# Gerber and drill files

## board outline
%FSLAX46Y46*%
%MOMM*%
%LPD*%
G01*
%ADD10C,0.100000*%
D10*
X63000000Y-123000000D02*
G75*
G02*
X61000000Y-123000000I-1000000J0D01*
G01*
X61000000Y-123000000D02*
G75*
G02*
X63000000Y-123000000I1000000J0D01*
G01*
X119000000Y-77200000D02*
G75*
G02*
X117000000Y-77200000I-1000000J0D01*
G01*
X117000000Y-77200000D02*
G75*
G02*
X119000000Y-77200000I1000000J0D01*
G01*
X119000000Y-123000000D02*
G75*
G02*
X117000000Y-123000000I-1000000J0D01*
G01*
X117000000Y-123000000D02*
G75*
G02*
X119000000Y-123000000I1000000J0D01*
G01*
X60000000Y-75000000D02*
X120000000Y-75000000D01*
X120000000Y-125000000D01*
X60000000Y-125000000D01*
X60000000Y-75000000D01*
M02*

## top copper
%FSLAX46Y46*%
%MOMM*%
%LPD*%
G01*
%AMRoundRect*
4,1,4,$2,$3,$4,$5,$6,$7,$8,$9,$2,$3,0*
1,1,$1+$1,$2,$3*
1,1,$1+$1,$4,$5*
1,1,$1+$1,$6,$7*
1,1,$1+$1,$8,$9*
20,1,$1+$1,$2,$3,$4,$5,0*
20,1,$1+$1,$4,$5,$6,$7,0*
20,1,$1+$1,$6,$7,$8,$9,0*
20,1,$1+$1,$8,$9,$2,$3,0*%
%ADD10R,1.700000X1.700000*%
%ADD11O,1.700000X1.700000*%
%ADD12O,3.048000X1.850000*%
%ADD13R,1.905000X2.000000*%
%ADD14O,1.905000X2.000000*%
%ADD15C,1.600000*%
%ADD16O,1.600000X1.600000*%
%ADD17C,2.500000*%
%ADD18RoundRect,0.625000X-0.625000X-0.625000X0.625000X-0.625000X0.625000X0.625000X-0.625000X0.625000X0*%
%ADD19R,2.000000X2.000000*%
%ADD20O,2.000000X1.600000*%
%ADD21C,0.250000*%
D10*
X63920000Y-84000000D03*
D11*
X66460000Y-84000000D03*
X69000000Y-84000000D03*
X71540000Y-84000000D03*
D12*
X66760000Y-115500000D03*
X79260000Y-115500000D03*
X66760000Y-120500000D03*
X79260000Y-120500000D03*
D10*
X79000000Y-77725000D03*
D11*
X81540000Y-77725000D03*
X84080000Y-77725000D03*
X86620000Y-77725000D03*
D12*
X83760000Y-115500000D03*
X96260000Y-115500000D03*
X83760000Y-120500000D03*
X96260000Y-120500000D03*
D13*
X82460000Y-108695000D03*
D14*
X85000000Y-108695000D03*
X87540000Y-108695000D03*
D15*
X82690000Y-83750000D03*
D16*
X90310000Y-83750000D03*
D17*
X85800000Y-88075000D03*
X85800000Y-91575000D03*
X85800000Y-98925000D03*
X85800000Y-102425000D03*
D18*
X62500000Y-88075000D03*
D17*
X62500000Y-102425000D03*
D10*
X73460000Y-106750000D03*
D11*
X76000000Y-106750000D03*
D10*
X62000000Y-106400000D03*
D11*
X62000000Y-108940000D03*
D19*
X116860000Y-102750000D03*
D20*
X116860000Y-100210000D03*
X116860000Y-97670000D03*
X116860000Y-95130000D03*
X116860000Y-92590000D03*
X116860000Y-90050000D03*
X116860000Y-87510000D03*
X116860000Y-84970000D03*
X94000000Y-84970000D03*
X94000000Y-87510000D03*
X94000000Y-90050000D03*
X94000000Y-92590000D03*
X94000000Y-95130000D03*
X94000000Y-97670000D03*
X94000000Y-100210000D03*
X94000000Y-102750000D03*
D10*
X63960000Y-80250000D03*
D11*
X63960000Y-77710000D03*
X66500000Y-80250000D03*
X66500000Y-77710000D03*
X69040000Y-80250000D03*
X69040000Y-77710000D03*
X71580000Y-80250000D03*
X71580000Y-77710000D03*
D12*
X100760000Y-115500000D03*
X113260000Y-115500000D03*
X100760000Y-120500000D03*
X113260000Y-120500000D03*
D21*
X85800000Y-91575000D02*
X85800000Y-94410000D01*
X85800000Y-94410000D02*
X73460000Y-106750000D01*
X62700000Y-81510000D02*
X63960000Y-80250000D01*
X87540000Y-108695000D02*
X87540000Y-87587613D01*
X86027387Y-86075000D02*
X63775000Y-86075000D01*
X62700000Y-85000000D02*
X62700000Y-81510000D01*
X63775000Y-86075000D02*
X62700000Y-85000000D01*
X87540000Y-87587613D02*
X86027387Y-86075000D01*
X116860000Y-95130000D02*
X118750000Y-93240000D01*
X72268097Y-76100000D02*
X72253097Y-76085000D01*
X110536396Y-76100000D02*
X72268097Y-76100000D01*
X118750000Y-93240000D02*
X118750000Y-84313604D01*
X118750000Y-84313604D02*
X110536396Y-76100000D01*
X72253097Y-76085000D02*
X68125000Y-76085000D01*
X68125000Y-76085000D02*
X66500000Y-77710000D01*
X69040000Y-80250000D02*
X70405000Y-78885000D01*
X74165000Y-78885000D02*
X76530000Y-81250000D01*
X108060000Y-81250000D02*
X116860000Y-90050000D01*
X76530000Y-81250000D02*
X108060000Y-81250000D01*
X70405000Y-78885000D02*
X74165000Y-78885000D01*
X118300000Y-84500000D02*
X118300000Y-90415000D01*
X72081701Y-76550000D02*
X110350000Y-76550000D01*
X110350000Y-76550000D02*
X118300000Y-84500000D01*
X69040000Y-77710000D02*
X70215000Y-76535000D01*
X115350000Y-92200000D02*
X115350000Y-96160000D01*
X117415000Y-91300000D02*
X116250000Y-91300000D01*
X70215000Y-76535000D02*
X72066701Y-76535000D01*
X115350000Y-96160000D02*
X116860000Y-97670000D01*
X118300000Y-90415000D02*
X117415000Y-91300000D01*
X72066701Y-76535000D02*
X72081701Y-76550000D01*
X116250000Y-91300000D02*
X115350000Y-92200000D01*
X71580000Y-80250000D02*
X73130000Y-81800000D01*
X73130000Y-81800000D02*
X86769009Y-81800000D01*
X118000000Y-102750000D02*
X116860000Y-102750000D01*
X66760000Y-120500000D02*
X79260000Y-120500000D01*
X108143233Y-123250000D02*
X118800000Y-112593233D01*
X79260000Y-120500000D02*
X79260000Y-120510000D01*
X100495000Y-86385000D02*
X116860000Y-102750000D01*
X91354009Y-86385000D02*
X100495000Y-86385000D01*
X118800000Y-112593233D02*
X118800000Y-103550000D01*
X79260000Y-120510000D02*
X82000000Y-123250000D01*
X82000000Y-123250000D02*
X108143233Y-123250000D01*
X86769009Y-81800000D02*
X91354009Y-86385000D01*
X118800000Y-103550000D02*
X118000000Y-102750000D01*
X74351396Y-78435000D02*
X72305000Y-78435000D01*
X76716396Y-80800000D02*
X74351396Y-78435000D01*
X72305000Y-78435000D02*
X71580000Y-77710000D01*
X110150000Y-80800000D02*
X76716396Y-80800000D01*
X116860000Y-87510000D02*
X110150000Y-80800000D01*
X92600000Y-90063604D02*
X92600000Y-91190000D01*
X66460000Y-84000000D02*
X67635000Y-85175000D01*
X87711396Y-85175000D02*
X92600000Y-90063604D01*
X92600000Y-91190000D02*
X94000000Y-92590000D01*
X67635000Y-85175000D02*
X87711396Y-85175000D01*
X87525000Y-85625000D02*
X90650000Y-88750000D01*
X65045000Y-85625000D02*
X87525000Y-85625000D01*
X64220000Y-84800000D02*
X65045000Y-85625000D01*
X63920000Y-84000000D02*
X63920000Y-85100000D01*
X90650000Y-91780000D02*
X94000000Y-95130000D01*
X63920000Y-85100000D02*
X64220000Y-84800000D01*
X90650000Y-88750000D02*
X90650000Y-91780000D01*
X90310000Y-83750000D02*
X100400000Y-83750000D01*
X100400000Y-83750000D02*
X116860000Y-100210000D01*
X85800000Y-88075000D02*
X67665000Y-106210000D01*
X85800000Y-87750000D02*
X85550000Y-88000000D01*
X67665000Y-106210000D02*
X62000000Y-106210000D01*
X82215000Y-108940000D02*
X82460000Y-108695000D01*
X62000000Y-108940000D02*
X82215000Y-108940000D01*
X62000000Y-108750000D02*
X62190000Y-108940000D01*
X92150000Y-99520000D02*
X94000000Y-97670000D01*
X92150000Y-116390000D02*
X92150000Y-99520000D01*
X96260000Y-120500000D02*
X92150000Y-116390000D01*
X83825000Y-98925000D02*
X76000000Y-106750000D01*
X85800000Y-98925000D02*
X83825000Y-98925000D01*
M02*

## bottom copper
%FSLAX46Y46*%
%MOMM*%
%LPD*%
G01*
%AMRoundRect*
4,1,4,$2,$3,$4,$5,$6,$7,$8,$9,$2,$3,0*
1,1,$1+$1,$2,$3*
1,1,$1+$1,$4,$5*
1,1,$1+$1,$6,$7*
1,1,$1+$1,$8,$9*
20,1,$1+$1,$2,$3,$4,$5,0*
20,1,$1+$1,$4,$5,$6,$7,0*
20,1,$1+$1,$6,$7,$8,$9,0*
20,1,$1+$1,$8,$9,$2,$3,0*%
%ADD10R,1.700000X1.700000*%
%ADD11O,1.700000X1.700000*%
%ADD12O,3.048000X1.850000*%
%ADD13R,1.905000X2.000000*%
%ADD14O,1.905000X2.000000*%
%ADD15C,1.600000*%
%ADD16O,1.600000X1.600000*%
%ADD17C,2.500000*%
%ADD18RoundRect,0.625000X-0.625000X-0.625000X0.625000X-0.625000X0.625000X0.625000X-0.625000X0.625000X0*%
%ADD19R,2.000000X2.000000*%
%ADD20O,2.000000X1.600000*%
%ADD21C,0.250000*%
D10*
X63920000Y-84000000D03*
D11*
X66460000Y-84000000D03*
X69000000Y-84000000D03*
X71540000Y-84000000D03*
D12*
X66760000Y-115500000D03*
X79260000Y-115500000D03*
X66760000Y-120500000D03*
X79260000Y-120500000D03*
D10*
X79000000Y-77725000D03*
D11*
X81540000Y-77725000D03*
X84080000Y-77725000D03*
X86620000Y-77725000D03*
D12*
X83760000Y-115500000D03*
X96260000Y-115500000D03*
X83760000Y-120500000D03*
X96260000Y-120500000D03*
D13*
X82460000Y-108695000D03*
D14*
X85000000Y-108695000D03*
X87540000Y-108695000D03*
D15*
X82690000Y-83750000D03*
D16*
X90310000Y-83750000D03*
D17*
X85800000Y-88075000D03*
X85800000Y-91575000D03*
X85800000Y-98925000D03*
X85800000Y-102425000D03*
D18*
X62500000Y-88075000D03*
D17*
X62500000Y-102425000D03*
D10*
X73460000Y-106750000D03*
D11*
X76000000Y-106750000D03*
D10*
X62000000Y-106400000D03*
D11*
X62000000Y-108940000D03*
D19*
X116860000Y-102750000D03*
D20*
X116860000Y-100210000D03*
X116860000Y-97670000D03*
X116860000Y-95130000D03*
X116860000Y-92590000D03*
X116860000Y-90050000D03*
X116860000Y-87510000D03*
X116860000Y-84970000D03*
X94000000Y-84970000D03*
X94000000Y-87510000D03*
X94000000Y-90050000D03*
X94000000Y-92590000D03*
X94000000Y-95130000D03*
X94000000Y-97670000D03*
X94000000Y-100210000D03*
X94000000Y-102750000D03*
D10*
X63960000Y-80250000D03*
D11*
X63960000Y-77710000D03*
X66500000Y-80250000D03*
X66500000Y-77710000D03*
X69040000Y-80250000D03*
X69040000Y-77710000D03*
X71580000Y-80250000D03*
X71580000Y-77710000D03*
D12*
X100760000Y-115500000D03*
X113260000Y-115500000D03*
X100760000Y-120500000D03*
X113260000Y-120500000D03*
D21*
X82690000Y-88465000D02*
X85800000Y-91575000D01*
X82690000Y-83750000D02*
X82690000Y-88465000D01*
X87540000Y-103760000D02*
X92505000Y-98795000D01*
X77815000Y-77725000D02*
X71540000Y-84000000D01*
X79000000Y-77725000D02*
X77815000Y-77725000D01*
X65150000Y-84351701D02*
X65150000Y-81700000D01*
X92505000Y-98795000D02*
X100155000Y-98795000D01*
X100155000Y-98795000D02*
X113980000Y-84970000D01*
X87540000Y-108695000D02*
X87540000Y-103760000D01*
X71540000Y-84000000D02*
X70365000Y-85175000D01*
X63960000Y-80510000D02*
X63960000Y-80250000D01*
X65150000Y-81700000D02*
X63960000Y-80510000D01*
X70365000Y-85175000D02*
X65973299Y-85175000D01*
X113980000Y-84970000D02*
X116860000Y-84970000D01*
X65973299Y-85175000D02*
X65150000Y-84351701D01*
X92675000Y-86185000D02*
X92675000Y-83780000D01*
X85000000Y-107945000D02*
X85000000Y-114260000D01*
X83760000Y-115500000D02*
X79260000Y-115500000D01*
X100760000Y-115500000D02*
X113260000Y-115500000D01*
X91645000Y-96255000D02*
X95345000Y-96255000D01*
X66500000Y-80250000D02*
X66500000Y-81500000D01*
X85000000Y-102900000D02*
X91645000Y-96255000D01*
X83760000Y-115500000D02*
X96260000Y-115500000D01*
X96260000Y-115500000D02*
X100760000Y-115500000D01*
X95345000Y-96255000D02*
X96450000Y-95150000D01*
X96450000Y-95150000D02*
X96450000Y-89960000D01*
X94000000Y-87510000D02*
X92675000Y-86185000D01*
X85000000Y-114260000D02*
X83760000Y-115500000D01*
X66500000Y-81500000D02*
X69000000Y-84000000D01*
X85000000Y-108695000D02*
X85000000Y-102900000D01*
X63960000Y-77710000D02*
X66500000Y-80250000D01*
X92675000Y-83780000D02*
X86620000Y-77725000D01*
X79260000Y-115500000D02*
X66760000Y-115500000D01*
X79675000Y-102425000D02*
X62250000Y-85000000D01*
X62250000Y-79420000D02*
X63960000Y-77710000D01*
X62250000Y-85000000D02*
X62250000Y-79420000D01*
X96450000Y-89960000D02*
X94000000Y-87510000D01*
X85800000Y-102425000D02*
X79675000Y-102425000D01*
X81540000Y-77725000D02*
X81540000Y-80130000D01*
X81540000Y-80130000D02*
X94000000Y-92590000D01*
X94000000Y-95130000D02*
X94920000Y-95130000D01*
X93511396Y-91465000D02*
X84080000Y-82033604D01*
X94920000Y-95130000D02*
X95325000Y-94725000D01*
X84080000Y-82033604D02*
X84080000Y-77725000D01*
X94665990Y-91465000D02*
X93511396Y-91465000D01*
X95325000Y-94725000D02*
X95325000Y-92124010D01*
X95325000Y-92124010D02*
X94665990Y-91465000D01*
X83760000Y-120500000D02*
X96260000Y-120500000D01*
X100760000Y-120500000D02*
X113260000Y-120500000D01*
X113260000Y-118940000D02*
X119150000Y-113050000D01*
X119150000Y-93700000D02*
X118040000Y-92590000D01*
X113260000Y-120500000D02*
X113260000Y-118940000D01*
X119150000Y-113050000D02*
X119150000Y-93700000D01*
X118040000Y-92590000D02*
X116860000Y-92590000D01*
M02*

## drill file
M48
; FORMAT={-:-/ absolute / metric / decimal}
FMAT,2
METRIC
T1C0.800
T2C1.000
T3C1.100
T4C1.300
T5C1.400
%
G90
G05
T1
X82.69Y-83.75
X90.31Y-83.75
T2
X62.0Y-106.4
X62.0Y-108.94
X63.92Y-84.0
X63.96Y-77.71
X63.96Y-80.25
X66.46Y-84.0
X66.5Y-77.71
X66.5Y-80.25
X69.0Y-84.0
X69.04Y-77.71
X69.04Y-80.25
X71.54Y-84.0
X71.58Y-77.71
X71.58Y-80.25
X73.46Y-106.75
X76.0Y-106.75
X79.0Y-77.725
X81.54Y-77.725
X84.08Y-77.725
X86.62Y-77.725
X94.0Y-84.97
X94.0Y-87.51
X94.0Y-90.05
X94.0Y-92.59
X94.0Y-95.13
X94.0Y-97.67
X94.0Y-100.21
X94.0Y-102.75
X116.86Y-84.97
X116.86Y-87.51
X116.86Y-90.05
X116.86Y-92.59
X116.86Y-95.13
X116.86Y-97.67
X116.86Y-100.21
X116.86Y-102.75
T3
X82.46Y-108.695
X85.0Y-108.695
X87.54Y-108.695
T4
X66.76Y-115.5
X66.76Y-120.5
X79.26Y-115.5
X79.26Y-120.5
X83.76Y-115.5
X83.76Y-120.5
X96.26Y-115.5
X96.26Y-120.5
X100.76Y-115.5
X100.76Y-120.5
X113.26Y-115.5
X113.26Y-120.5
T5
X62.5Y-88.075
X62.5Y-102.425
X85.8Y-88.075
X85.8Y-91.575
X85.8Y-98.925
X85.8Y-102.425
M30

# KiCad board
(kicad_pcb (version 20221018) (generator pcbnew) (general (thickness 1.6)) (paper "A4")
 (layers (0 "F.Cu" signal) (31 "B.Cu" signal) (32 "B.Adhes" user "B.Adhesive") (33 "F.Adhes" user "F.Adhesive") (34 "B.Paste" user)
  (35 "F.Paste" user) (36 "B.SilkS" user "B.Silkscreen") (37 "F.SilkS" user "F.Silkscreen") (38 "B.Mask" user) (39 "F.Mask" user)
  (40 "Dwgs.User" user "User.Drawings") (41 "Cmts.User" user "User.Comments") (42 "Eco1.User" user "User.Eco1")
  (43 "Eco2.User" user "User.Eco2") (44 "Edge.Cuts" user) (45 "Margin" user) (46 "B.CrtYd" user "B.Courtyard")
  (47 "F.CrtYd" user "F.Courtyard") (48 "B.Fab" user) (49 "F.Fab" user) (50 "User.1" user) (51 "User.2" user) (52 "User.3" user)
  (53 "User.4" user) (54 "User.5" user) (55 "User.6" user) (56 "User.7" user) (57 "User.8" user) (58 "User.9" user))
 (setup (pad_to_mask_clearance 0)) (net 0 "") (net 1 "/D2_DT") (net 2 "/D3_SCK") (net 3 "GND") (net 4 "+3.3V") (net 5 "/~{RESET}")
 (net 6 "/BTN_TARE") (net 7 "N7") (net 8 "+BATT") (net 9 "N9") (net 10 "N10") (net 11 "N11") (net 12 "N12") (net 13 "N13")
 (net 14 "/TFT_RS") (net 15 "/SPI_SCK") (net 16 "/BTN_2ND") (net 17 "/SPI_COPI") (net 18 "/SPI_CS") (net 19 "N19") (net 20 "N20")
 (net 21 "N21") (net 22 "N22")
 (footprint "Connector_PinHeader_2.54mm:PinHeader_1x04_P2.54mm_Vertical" (layer "F.Cu") (at 63.92 84 90)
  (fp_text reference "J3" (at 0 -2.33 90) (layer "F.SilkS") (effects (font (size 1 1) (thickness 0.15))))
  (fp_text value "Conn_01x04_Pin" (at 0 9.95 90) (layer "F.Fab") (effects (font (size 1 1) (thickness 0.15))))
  (pad "1" thru_hole rect (at 0 0 90) (size 1.7 1.7) (drill 1) (layers "*.Cu" "*.Mask") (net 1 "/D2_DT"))
  (pad "2" thru_hole oval (at 0 2.54 90) (size 1.7 1.7) (drill 1) (layers "*.Cu" "*.Mask") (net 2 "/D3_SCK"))
  (pad "3" thru_hole oval (at 0 5.08 90) (size 1.7 1.7) (drill 1) (layers "*.Cu" "*.Mask") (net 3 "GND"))
  (pad "4" thru_hole oval (at 0 7.62 90) (size 1.7 1.7) (drill 1) (layers "*.Cu" "*.Mask") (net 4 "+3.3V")))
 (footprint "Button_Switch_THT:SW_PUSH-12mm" (layer "F.Cu") (at 66.76 115.5)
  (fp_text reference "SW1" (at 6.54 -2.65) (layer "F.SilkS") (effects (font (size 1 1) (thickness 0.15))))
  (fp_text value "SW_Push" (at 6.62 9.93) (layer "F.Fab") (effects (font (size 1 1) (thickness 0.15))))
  (pad "1" thru_hole oval (at 0 0) (size 3.048 1.85) (drill 1.3) (layers "*.Cu" "*.Mask") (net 3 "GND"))
  (pad "1" thru_hole oval (at 12.5 0) (size 3.048 1.85) (drill 1.3) (layers "*.Cu" "*.Mask") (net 3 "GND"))
  (pad "2" thru_hole oval (at 0 5) (size 3.048 1.85) (drill 1.3) (layers "*.Cu" "*.Mask") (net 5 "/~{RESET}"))
  (pad "2" thru_hole oval (at 12.5 5) (size 3.048 1.85) (drill 1.3) (layers "*.Cu" "*.Mask") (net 5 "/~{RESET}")))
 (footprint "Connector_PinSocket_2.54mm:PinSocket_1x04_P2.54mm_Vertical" (layer "F.Cu") (at 79 77.725 90)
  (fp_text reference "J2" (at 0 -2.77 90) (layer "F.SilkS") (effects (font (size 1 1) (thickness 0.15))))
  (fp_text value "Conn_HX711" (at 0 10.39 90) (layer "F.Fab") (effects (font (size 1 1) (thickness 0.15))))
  (pad "1" thru_hole rect (at 0 0 90) (size 1.7 1.7) (drill 1) (layers "*.Cu" "*.Mask") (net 4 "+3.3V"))
  (pad "2" thru_hole oval (at 0 2.54 90) (size 1.7 1.7) (drill 1) (layers "*.Cu" "*.Mask") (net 2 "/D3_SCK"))
  (pad "3" thru_hole oval (at 0 5.08 90) (size 1.7 1.7) (drill 1) (layers "*.Cu" "*.Mask") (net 1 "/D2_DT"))
  (pad "4" thru_hole oval (at 0 7.62 90) (size 1.7 1.7) (drill 1) (layers "*.Cu" "*.Mask") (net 3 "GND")))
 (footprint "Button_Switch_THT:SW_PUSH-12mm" (layer "F.Cu") (at 83.76 115.5)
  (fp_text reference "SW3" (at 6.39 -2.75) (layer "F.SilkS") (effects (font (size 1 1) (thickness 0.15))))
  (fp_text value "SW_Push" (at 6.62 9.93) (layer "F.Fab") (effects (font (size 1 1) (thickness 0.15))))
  (pad "1" thru_hole oval (at 0 0) (size 3.048 1.85) (drill 1.3) (layers "*.Cu" "*.Mask") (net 3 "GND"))
  (pad "1" thru_hole oval (at 12.5 0) (size 3.048 1.85) (drill 1.3) (layers "*.Cu" "*.Mask") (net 3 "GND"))
  (pad "2" thru_hole oval (at 0 5) (size 3.048 1.85) (drill 1.3) (layers "*.Cu" "*.Mask") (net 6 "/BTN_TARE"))
  (pad "2" thru_hole oval (at 12.5 5) (size 3.048 1.85) (drill 1.3) (layers "*.Cu" "*.Mask") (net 6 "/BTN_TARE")))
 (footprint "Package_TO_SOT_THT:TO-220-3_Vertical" (layer "F.Cu") (at 82.46 108.695)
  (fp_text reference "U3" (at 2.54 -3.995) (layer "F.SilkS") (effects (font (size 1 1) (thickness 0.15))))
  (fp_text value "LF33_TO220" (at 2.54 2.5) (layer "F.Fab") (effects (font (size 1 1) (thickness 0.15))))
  (pad "1" thru_hole rect (at 0 0) (size 1.905 2) (drill 1.1) (layers "*.Cu" "*.Mask") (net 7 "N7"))
  (pad "2" thru_hole oval (at 2.54 0) (size 1.905 2) (drill 1.1) (layers "*.Cu" "*.Mask") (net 3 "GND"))
  (pad "3" thru_hole oval (at 5.08 0) (size 1.905 2) (drill 1.1) (layers "*.Cu" "*.Mask") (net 4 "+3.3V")))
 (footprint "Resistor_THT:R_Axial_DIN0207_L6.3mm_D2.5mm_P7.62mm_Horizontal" (layer "F.Cu") (at 82.69 83.75)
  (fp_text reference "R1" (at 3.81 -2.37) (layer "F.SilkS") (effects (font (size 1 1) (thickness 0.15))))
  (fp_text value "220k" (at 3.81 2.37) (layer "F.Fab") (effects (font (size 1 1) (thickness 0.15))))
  (pad "1" thru_hole circle (at 0 0) (size 1.6 1.6) (drill 0.8) (layers "*.Cu" "*.Mask") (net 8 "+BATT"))
  (pad "2" thru_hole oval (at 7.62 0) (size 1.6 1.6) (drill 0.8) (layers "*.Cu" "*.Mask") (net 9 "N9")))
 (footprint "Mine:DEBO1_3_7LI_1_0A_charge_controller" (layer "F.Cu") (at 60.8 93.575)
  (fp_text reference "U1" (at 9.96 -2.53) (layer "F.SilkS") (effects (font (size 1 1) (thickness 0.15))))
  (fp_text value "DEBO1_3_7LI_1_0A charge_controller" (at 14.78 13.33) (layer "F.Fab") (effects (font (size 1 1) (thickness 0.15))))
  (pad "1" thru_hole circle (at 25 -5.5) (size 2.5 2.5) (drill 1.4) (layers "*.Cu" "*.Mask") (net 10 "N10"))
  (pad "2" thru_hole circle (at 25 -2) (size 2.5 2.5) (drill 1.4) (layers "*.Cu" "*.Mask") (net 8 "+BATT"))
  (pad "3" thru_hole circle (at 25 5.35) (size 2.5 2.5) (drill 1.4) (layers "*.Cu" "*.Mask") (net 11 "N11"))
  (pad "4" thru_hole circle (at 25 8.85) (size 2.5 2.5) (drill 1.4) (layers "*.Cu" "*.Mask") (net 3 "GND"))
  (pad "5" thru_hole roundrect (at 1.7 -5.5) (size 2.5 2.5) (drill 1.4) (layers "*.Cu" "*.Mask") (roundrect_rratio 0.25) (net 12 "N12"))
  (pad "6" thru_hole circle (at 1.7 8.85) (size 2.5 2.5) (drill 1.4) (layers "*.Cu" "*.Mask") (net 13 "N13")))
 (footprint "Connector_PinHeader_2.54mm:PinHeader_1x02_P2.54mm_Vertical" (layer "F.Cu") (at 73.46 106.75 90)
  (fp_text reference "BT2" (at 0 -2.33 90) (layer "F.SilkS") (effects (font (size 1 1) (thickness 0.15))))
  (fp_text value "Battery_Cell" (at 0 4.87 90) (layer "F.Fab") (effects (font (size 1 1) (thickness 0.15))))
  (pad "1" thru_hole rect (at 0 0 90) (size 1.7 1.7) (drill 1) (layers "*.Cu" "*.Mask") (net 8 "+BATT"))
  (pad "2" thru_hole oval (at 0 2.54 90) (size 1.7 1.7) (drill 1) (layers "*.Cu" "*.Mask") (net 11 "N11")))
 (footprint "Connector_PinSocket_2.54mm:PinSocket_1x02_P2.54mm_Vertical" (layer "F.Cu") (at 62 106.4)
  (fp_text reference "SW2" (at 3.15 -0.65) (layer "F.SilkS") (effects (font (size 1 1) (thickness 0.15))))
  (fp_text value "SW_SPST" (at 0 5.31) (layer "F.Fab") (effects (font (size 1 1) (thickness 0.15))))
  (pad "1" thru_hole rect (at 0 0) (size 1.7 1.7) (drill 1) (layers "*.Cu" "*.Mask") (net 10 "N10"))
  (pad "2" thru_hole oval (at 0 2.54) (size 1.7 1.7) (drill 1) (layers "*.Cu" "*.Mask") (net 7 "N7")))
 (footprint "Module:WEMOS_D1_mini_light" (layer "F.Cu") (at 116.86 102.75 180)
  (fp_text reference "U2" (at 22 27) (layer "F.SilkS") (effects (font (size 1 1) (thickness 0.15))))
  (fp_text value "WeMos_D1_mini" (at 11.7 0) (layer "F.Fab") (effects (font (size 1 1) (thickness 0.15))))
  (pad "1" thru_hole rect (at 0 0 180) (size 2 2) (drill 1) (layers "*.Cu" "*.Mask") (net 5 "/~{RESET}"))
  (pad "2" thru_hole oval (at 0 2.54 180) (size 2 1.6) (drill 1) (layers "*.Cu" "*.Mask") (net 9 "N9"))
  (pad "3" thru_hole oval (at 0 5.08 180) (size 2 1.6) (drill 1) (layers "*.Cu" "*.Mask") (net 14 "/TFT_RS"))
  (pad "4" thru_hole oval (at 0 7.62 180) (size 2 1.6) (drill 1) (layers "*.Cu" "*.Mask") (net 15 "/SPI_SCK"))
  (pad "5" thru_hole oval (at 0 10.16 180) (size 2 1.6) (drill 1) (layers "*.Cu" "*.Mask") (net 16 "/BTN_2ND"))
  (pad "6" thru_hole oval (at 0 12.7 180) (size 2 1.6) (drill 1) (layers "*.Cu" "*.Mask") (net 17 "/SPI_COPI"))
  (pad "7" thru_hole oval (at 0 15.24 180) (size 2 1.6) (drill 1) (layers "*.Cu" "*.Mask") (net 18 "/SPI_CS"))
  (pad "8" thru_hole oval (at 0 17.78 180) (size 2 1.6) (drill 1) (layers "*.Cu" "*.Mask") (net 4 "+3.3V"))
  (pad "9" thru_hole oval (at 22.86 17.78 180) (size 2 1.6) (drill 1) (layers "*.Cu" "*.Mask") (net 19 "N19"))
  (pad "10" thru_hole oval (at 22.86 15.24 180) (size 2 1.6) (drill 1) (layers "*.Cu" "*.Mask") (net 3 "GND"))
  (pad "11" thru_hole oval (at 22.86 12.7 180) (size 2 1.6) (drill 1) (layers "*.Cu" "*.Mask") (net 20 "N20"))
  (pad "12" thru_hole oval (at 22.86 10.16 180) (size 2 1.6) (drill 1) (layers "*.Cu" "*.Mask") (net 2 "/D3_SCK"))
  (pad "13" thru_hole oval (at 22.86 7.62 180) (size 2 1.6) (drill 1) (layers "*.Cu" "*.Mask") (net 1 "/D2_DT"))
  (pad "14" thru_hole oval (at 22.86 5.08 180) (size 2 1.6) (drill 1) (layers "*.Cu" "*.Mask") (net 6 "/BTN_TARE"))
  (pad "15" thru_hole oval (at 22.86 2.54 180) (size 2 1.6) (drill 1) (layers "*.Cu" "*.Mask") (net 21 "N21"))
  (pad "16" thru_hole oval (at 22.86 0 180) (size 2 1.6) (drill 1) (layers "*.Cu" "*.Mask") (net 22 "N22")))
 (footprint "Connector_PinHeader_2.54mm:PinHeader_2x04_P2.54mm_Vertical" (layer "F.Cu") (at 63.96 80.25 90)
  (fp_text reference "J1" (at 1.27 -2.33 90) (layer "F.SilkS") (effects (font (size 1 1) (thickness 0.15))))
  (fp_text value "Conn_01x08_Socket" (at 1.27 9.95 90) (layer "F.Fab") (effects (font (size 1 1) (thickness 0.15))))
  (pad "1" thru_hole rect (at 0 0 90) (size 1.7 1.7) (drill 1) (layers "*.Cu" "*.Mask") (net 4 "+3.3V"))
  (pad "2" thru_hole oval (at 2.54 0 90) (size 1.7 1.7) (drill 1) (layers "*.Cu" "*.Mask") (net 3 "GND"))
  (pad "3" thru_hole oval (at 0 2.54 90) (size 1.7 1.7) (drill 1) (layers "*.Cu" "*.Mask") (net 3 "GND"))
  (pad "4" thru_hole oval (at 2.54 2.54 90) (size 1.7 1.7) (drill 1) (layers "*.Cu" "*.Mask") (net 15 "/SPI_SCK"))
  (pad "5" thru_hole oval (at 0 5.08 90) (size 1.7 1.7) (drill 1) (layers "*.Cu" "*.Mask") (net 17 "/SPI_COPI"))
  (pad "6" thru_hole oval (at 2.54 5.08 90) (size 1.7 1.7) (drill 1) (layers "*.Cu" "*.Mask") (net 14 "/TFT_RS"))
  (pad "7" thru_hole oval (at 0 7.62 90) (size 1.7 1.7) (drill 1) (layers "*.Cu" "*.Mask") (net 5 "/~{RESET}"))
  (pad "8" thru_hole oval (at 2.54 7.62 90) (size 1.7 1.7) (drill 1) (layers "*.Cu" "*.Mask") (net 18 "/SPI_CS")))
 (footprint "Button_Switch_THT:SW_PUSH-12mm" (layer "F.Cu") (at 100.76 115.5)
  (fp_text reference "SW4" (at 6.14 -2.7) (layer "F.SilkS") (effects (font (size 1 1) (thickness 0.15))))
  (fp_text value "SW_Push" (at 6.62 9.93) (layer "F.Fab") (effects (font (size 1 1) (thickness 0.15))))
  (pad "1" thru_hole oval (at 0 0) (size 3.048 1.85) (drill 1.3) (layers "*.Cu" "*.Mask") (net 3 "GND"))
  (pad "1" thru_hole oval (at 12.5 0) (size 3.048 1.85) (drill 1.3) (layers "*.Cu" "*.Mask") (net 3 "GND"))
  (pad "2" thru_hole oval (at 0 5) (size 3.048 1.85) (drill 1.3) (layers "*.Cu" "*.Mask") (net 16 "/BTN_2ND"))
  (pad "2" thru_hole oval (at 12.5 5) (size 3.048 1.85) (drill 1.3) (layers "*.Cu" "*.Mask") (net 16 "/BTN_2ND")))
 (gr_circle (center 62 123) (end 62.8 123.6) (stroke (width 0.1) (type default)) (fill none) (layer "Edge.Cuts"))
 (gr_circle (center 118 77.2) (end 118.8 77.8) (stroke (width 0.1) (type default)) (fill none) (layer "Edge.Cuts"))
 (gr_circle (center 118 123) (end 118.8 123.6) (stroke (width 0.1) (type default)) (fill none) (layer "Edge.Cuts"))
 (gr_rect (start 60 75) (end 120 125) (stroke (width 0.1) (type default)) (fill none) (layer "Edge.Cuts"))
 (segment (start 85.8 91.575) (end 85.8 94.41) (width 0.25) (layer "F.Cu") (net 8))
 (segment (start 85.8 94.41) (end 73.46 106.75) (width 0.25) (layer "F.Cu") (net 8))
 (segment (start 82.69 88.465) (end 85.8 91.575) (width 0.25) (layer "B.Cu") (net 8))
 (segment (start 82.69 83.75) (end 82.69 88.465) (width 0.25) (layer "B.Cu") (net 8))
 (segment (start 62.7 81.51) (end 63.96 80.25) (width 0.25) (layer "F.Cu") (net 4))
 (segment (start 87.54 108.695) (end 87.54 87.587613) (width 0.25) (layer "F.Cu") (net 4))
 (segment (start 86.027387 86.075) (end 63.775 86.075) (width 0.25) (layer "F.Cu") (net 4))
 (segment (start 62.7 85) (end 62.7 81.51) (width 0.25) (layer "F.Cu") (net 4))
 (segment (start 63.775 86.075) (end 62.7 85) (width 0.25) (layer "F.Cu") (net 4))
 (segment (start 87.54 87.587613) (end 86.027387 86.075) (width 0.25) (layer "F.Cu") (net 4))
 (segment (start 87.54 103.76) (end 92.505 98.795) (width 0.25) (layer "B.Cu") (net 4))
 (segment (start 77.815 77.725) (end 71.54 84) (width 0.25) (layer "B.Cu") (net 4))
 (segment (start 79 77.725) (end 77.815 77.725) (width 0.25) (layer "B.Cu") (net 4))
 (segment (start 65.15 84.351701) (end 65.15 81.7) (width 0.25) (layer "B.Cu") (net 4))
 (segment (start 92.505 98.795) (end 100.155 98.795) (width 0.25) (layer "B.Cu") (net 4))
 (segment (start 100.155 98.795) (end 113.98 84.97) (width 0.25) (layer "B.Cu") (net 4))
 (segment (start 87.54 108.695) (end 87.54 103.76) (width 0.25) (layer "B.Cu") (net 4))
 (segment (start 71.54 84) (end 70.365 85.175) (width 0.25) (layer "B.Cu") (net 4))
 (segment (start 63.96 80.51) (end 63.96 80.25) (width 0.25) (layer "B.Cu") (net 4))
 (segment (start 65.15 81.7) (end 63.96 80.51) (width 0.25) (layer "B.Cu") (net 4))
 (segment (start 70.365 85.175) (end 65.973299 85.175) (width 0.25) (layer "B.Cu") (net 4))
 (segment (start 113.98 84.97) (end 116.86 84.97) (width 0.25) (layer "B.Cu") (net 4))
 (segment (start 65.973299 85.175) (end 65.15 84.351701) (width 0.25) (layer "B.Cu") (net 4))
 (segment (start 92.675 86.185) (end 92.675 83.78) (width 0.25) (layer "B.Cu") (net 3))
 (segment (start 85 107.945) (end 85 114.26) (width 0.25) (layer "B.Cu") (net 3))
 (segment (start 83.76 115.5) (end 79.26 115.5) (width 0.25) (layer "B.Cu") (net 3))
 (segment (start 100.76 115.5) (end 113.26 115.5) (width 0.25) (layer "B.Cu") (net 3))
 (segment (start 91.645 96.255) (end 95.345 96.255) (width 0.25) (layer "B.Cu") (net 3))
 (segment (start 66.5 80.25) (end 66.5 81.5) (width 0.25) (layer "B.Cu") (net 3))
 (segment (start 85 102.9) (end 91.645 96.255) (width 0.25) (layer "B.Cu") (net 3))
 (segment (start 83.76 115.5) (end 96.26 115.5) (width 0.25) (layer "B.Cu") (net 3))
 (segment (start 96.26 115.5) (end 100.76 115.5) (width 0.25) (layer "B.Cu") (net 3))
 (segment (start 95.345 96.255) (end 96.45 95.15) (width 0.25) (layer "B.Cu") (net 3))
 (segment (start 96.45 95.15) (end 96.45 89.96) (width 0.25) (layer "B.Cu") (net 3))
 (segment (start 94 87.51) (end 92.675 86.185) (width 0.25) (layer "B.Cu") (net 3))
 (segment (start 85 114.26) (end 83.76 115.5) (width 0.25) (layer "B.Cu") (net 3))
 (segment (start 66.5 81.5) (end 69 84) (width 0.25) (layer "B.Cu") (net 3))
 (segment (start 85 108.695) (end 85 102.9) (width 0.25) (layer "B.Cu") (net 3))
 (segment (start 63.96 77.71) (end 66.5 80.25) (width 0.25) (layer "B.Cu") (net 3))
 (segment (start 92.675 83.78) (end 86.62 77.725) (width 0.25) (layer "B.Cu") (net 3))
 (segment (start 79.26 115.5) (end 66.76 115.5) (width 0.25) (layer "B.Cu") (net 3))
 (segment (start 79.675 102.425) (end 62.25 85) (width 0.25) (layer "B.Cu") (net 3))
 (segment (start 62.25 79.42) (end 63.96 77.71) (width 0.25) (layer "B.Cu") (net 3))
 (segment (start 62.25 85) (end 62.25 79.42) (width 0.25) (layer "B.Cu") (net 3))
 (segment (start 96.45 89.96) (end 94 87.51) (width 0.25) (layer "B.Cu") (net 3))
 (segment (start 85.8 102.425) (end 79.675 102.425) (width 0.25) (layer "B.Cu") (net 3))
 (segment (start 116.86 95.13) (end 118.75 93.24) (width 0.25) (layer "F.Cu") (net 15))
 (segment (start 72.268097 76.1) (end 72.253097 76.085) (width 0.25) (layer "F.Cu") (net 15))
 (segment (start 110.536396 76.1) (end 72.268097 76.1) (width 0.25) (layer "F.Cu") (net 15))
 (segment (start 118.75 93.24) (end 118.75 84.313604) (width 0.25) (layer "F.Cu") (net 15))
 (segment (start 118.75 84.313604) (end 110.536396 76.1) (width 0.25) (layer "F.Cu") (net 15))
 (segment (start 72.253097 76.085) (end 68.125 76.085) (width 0.25) (layer "F.Cu") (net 15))
 (segment (start 68.125 76.085) (end 66.5 77.71) (width 0.25) (layer "F.Cu") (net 15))
 (segment (start 69.04 80.25) (end 70.405 78.885) (width 0.25) (layer "F.Cu") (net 17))
 (segment (start 74.165 78.885) (end 76.53 81.25) (width 0.25) (layer "F.Cu") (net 17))
 (segment (start 108.06 81.25) (end 116.86 90.05) (width 0.25) (layer "F.Cu") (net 17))
 (segment (start 76.53 81.25) (end 108.06 81.25) (width 0.25) (layer "F.Cu") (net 17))
 (segment (start 70.405 78.885) (end 74.165 78.885) (width 0.25) (layer "F.Cu") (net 17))
 (segment (start 118.3 84.5) (end 118.3 90.415) (width 0.25) (layer "F.Cu") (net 14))
 (segment (start 72.081701 76.55) (end 110.35 76.55) (width 0.25) (layer "F.Cu") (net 14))
 (segment (start 110.35 76.55) (end 118.3 84.5) (width 0.25) (layer "F.Cu") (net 14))
 (segment (start 69.04 77.71) (end 70.215 76.535) (width 0.25) (layer "F.Cu") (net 14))
 (segment (start 115.35 92.2) (end 115.35 96.16) (width 0.25) (layer "F.Cu") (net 14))
 (segment (start 117.415 91.3) (end 116.25 91.3) (width 0.25) (layer "F.Cu") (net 14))
 (segment (start 70.215 76.535) (end 72.066701 76.535) (width 0.25) (layer "F.Cu") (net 14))
 (segment (start 115.35 96.16) (end 116.86 97.67) (width 0.25) (layer "F.Cu") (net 14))
 (segment (start 118.3 90.415) (end 117.415 91.3) (width 0.25) (layer "F.Cu") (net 14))
 (segment (start 72.066701 76.535) (end 72.081701 76.55) (width 0.25) (layer "F.Cu") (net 14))
 (segment (start 116.25 91.3) (end 115.35 92.2) (width 0.25) (layer "F.Cu") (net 14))
 (segment (start 71.58 80.25) (end 73.13 81.8) (width 0.25) (layer "F.Cu") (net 5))
 (segment (start 73.13 81.8) (end 86.769009 81.8) (width 0.25) (layer "F.Cu") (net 5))
 (segment (start 118 102.75) (end 116.86 102.75) (width 0.25) (layer "F.Cu") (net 5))
 (segment (start 66.76 120.5) (end 79.26 120.5) (width 0.25) (layer "F.Cu") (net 5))
 (segment (start 108.143233 123.25) (end 118.8 112.593233) (width 0.25) (layer "F.Cu") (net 5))
 (segment (start 79.26 120.5) (end 79.26 120.51) (width 0.25) (layer "F.Cu") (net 5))
 (segment (start 100.495 86.385) (end 116.86 102.75) (width 0.25) (layer "F.Cu") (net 5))
 (segment (start 91.354009 86.385) (end 100.495 86.385) (width 0.25) (layer "F.Cu") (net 5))
 (segment (start 118.8 112.593233) (end 118.8 103.55) (width 0.25) (layer "F.Cu") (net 5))
 (segment (start 79.26 120.51) (end 82 123.25) (width 0.25) (layer "F.Cu") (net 5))
 (segment (start 82 123.25) (end 108.143233 123.25) (width 0.25) (layer "F.Cu") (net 5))
 (segment (start 86.769009 81.8) (end 91.354009 86.385) (width 0.25) (layer "F.Cu") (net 5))
 (segment (start 118.8 103.55) (end 118 102.75) (width 0.25) (layer "F.Cu") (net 5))
 (segment (start 74.351396 78.435) (end 72.305 78.435) (width 0.25) (layer "F.Cu") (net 18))
 (segment (start 76.716396 80.8) (end 74.351396 78.435) (width 0.25) (layer "F.Cu") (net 18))
 (segment (start 72.305 78.435) (end 71.58 77.71) (width 0.25) (layer "F.Cu") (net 18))
 (segment (start 110.15 80.8) (end 76.716396 80.8) (width 0.25) (layer "F.Cu") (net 18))
 (segment (start 116.86 87.51) (end 110.15 80.8) (width 0.25) (layer "F.Cu") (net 18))
 (segment (start 92.6 90.063604) (end 92.6 91.19) (width 0.25) (layer "F.Cu") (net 2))
 (segment (start 66.46 84) (end 67.635 85.175) (width 0.25) (layer "F.Cu") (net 2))
 (segment (start 87.711396 85.175) (end 92.6 90.063604) (width 0.25) (layer "F.Cu") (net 2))
 (segment (start 92.6 91.19) (end 94 92.59) (width 0.25) (layer "F.Cu") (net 2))
 (segment (start 67.635 85.175) (end 87.711396 85.175) (width 0.25) (layer "F.Cu") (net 2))
 (segment (start 81.54 77.725) (end 81.54 80.13) (width 0.25) (layer "B.Cu") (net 2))
 (segment (start 81.54 80.13) (end 94 92.59) (width 0.25) (layer "B.Cu") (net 2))
 (segment (start 87.525 85.625) (end 90.65 88.75) (width 0.25) (layer "F.Cu") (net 1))
 (segment (start 65.045 85.625) (end 87.525 85.625) (width 0.25) (layer "F.Cu") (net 1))
 (segment (start 64.22 84.8) (end 65.045 85.625) (width 0.25) (layer "F.Cu") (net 1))
 (segment (start 63.92 84) (end 63.92 85.1) (width 0.25) (layer "F.Cu") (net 1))
 (segment (start 90.65 91.78) (end 94 95.13) (width 0.25) (layer "F.Cu") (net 1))
 (segment (start 63.92 85.1) (end 64.22 84.8) (width 0.25) (layer "F.Cu") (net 1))
 (segment (start 90.65 88.75) (end 90.65 91.78) (width 0.25) (layer "F.Cu") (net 1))
 (segment (start 94 95.13) (end 94.92 95.13) (width 0.25) (layer "B.Cu") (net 1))
 (segment (start 93.511396 91.465) (end 84.08 82.033604) (width 0.25) (layer "B.Cu") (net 1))
 (segment (start 94.92 95.13) (end 95.325 94.725) (width 0.25) (layer "B.Cu") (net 1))
 (segment (start 84.08 82.033604) (end 84.08 77.725) (width 0.25) (layer "B.Cu") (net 1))
 (segment (start 94.66599 91.465) (end 93.511396 91.465) (width 0.25) (layer "B.Cu") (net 1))
 (segment (start 95.325 94.725) (end 95.325 92.12401) (width 0.25) (layer "B.Cu") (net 1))
 (segment (start 95.325 92.12401) (end 94.66599 91.465) (width 0.25) (layer "B.Cu") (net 1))
 (segment (start 90.31 83.75) (end 100.4 83.75) (width 0.25) (layer "F.Cu") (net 9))
 (segment (start 100.4 83.75) (end 116.86 100.21) (width 0.25) (layer "F.Cu") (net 9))
 (segment (start 85.8 88.075) (end 67.665 106.21) (width 0.25) (layer "F.Cu") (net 10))
 (segment (start 85.8 87.75) (end 85.55 88) (width 0.25) (layer "F.Cu") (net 10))
 (segment (start 67.665 106.21) (end 62 106.21) (width 0.25) (layer "F.Cu") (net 10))
 (segment (start 82.215 108.94) (end 82.46 108.695) (width 0.25) (layer "F.Cu") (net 7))
 (segment (start 62 108.94) (end 82.215 108.94) (width 0.25) (layer "F.Cu") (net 7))
 (segment (start 62 108.75) (end 62.19 108.94) (width 0.25) (layer "F.Cu") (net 7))
 (segment (start 92.15 99.52) (end 94 97.67) (width 0.25) (layer "F.Cu") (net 6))
 (segment (start 92.15 116.39) (end 92.15 99.52) (width 0.25) (layer "F.Cu") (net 6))
 (segment (start 96.26 120.5) (end 92.15 116.39) (width 0.25) (layer "F.Cu") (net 6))
 (segment (start 83.76 120.5) (end 96.26 120.5) (width 0.25) (layer "B.Cu") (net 6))
 (segment (start 100.76 120.5) (end 113.26 120.5) (width 0.25) (layer "B.Cu") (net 16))
 (segment (start 113.26 118.94) (end 119.15 113.05) (width 0.25) (layer "B.Cu") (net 16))
 (segment (start 119.15 93.7) (end 118.04 92.59) (width 0.25) (layer "B.Cu") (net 16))
 (segment (start 113.26 120.5) (end 113.26 118.94) (width 0.25) (layer "B.Cu") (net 16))
 (segment (start 119.15 113.05) (end 119.15 93.7) (width 0.25) (layer "B.Cu") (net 16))
 (segment (start 118.04 92.59) (end 116.86 92.59) (width 0.25) (layer "B.Cu") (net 16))
 (segment (start 83.825 98.925) (end 76 106.75) (width 0.25) (layer "F.Cu") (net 11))
 (segment (start 85.8 98.925) (end 83.825 98.925) (width 0.25) (layer "F.Cu") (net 11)))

